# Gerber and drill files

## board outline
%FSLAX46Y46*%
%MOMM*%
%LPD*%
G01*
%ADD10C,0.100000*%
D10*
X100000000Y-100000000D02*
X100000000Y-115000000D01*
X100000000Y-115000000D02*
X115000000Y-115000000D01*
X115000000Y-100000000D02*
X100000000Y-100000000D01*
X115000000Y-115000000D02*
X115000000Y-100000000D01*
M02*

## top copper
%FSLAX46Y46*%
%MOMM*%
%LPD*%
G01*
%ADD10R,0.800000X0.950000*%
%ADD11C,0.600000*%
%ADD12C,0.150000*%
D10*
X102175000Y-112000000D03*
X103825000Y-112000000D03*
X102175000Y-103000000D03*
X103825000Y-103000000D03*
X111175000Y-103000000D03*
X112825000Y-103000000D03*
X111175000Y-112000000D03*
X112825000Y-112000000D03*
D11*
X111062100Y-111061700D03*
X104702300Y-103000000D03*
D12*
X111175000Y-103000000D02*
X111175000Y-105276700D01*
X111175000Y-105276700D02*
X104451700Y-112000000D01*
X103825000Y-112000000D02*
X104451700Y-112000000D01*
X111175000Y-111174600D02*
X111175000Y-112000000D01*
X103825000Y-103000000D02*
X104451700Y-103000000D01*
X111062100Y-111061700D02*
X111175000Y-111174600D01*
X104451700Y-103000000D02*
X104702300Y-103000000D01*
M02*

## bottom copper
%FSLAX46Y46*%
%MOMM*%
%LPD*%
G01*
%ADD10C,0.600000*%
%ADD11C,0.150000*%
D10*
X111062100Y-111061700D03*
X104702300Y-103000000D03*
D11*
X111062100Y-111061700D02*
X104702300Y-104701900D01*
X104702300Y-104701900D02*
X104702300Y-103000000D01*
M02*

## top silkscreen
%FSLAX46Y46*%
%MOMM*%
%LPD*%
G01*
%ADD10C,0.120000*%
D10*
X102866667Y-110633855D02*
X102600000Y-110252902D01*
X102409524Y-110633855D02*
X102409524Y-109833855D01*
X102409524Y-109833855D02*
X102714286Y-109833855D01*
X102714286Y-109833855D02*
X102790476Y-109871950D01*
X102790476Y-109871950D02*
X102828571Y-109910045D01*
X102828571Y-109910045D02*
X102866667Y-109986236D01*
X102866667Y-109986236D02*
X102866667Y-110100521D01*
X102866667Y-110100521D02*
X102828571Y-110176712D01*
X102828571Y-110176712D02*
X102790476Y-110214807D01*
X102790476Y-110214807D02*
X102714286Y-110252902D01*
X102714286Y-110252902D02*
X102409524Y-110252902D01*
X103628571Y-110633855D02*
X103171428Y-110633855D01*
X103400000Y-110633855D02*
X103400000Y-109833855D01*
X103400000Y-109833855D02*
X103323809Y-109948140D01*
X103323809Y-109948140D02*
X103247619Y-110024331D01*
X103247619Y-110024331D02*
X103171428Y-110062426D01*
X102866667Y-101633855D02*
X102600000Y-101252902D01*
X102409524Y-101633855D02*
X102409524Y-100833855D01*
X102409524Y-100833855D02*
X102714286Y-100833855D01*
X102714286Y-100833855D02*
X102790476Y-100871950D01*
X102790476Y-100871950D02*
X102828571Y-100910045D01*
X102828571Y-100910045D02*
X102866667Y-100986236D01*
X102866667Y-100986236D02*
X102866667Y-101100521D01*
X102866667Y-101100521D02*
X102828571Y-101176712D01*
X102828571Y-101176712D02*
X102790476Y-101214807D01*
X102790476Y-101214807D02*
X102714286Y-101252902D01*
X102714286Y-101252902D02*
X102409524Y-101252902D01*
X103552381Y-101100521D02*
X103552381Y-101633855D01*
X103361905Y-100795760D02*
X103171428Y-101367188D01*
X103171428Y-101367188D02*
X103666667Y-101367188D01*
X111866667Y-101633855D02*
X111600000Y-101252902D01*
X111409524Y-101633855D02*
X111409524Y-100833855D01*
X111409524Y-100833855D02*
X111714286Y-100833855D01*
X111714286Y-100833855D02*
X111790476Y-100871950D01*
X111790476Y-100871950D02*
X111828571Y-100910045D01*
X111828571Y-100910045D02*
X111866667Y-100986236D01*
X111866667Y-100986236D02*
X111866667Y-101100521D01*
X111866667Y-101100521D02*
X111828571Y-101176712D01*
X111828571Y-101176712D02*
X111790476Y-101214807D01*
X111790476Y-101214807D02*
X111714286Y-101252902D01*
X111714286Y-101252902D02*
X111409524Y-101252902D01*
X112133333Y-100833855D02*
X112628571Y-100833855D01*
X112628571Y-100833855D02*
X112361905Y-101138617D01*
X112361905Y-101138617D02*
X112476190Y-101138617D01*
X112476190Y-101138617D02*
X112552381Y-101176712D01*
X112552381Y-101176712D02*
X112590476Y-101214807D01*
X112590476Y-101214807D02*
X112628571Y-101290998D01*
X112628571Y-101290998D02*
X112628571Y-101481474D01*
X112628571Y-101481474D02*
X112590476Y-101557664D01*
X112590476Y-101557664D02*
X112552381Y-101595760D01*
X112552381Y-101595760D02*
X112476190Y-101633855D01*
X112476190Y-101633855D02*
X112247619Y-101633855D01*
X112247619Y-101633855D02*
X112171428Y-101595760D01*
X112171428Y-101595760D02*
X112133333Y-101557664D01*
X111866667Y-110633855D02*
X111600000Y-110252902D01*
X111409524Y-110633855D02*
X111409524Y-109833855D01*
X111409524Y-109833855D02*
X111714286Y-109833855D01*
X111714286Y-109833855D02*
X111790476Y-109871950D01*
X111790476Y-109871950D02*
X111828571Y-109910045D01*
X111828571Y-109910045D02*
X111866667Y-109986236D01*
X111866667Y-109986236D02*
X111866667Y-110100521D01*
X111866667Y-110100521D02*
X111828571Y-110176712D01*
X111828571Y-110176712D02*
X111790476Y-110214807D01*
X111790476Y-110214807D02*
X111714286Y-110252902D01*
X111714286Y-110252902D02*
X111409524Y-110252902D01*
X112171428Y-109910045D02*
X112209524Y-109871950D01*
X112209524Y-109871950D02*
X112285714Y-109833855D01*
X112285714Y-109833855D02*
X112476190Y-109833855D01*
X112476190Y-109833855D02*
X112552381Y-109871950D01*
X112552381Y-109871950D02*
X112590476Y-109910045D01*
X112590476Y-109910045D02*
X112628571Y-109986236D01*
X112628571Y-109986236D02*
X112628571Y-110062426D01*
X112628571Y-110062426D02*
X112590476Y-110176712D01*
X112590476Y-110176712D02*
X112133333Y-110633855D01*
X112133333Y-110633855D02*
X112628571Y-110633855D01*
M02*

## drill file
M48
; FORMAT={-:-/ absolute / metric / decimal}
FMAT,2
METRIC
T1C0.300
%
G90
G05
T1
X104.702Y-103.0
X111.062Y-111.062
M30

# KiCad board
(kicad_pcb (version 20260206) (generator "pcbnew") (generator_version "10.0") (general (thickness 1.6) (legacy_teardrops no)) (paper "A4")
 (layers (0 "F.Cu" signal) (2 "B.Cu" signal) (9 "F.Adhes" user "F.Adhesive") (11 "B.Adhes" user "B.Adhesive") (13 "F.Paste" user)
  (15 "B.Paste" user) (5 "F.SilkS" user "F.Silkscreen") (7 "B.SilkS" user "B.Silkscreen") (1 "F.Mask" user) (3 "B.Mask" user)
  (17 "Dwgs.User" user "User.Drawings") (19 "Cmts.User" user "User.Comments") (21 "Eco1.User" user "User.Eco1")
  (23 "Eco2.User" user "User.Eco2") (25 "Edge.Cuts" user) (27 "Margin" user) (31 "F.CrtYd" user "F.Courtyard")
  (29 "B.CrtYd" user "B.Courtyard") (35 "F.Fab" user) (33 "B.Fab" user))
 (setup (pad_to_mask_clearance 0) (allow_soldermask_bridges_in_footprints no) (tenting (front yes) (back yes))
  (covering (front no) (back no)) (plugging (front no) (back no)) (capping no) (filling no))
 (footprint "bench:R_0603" (layer "F.Cu") (at 103 112)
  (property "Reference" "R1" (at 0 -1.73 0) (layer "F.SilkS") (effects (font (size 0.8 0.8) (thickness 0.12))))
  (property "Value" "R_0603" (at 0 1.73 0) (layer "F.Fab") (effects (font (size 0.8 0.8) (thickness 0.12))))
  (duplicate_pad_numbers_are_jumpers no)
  (pad "1" smd rect (at -0.825 0) (size 0.8 0.95) (layers "F.Cu" "F.Mask" "F.Paste"))
  (pad "2" smd rect (at 0.825 0) (size 0.8 0.95) (layers "F.Cu" "F.Mask" "F.Paste") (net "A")))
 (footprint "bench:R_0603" (layer "F.Cu") (at 103 103)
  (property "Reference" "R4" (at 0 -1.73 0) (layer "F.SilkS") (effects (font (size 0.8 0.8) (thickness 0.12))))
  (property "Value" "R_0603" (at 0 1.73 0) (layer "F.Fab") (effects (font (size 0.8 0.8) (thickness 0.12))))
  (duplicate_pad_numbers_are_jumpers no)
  (pad "1" smd rect (at -0.825 0) (size 0.8 0.95) (layers "F.Cu" "F.Mask" "F.Paste"))
  (pad "2" smd rect (at 0.825 0) (size 0.8 0.95) (layers "F.Cu" "F.Mask" "F.Paste") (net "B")))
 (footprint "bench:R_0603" (layer "F.Cu") (at 112 103)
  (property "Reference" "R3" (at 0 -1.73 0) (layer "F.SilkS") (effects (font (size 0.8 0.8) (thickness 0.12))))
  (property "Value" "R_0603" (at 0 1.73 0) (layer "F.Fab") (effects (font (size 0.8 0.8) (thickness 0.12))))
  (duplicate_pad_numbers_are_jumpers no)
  (pad "1" smd rect (at -0.825 0) (size 0.8 0.95) (layers "F.Cu" "F.Mask" "F.Paste") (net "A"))
  (pad "2" smd rect (at 0.825 0) (size 0.8 0.95) (layers "F.Cu" "F.Mask" "F.Paste")))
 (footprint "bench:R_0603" (layer "F.Cu") (at 112 112)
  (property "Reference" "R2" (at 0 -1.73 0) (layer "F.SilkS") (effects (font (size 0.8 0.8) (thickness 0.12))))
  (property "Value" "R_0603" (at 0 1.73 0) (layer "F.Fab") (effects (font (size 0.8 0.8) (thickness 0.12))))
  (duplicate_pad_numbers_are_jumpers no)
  (pad "1" smd rect (at -0.825 0) (size 0.8 0.95) (layers "F.Cu" "F.Mask" "F.Paste") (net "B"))
  (pad "2" smd rect (at 0.825 0) (size 0.8 0.95) (layers "F.Cu" "F.Mask" "F.Paste")))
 (gr_line (start 100 100) (end 100 115) (stroke (width 0.1) (type solid)) (layer "Edge.Cuts"))
 (gr_line (start 100 115) (end 115 115) (stroke (width 0.1) (type solid)) (layer "Edge.Cuts"))
 (gr_line (start 115 100) (end 100 100) (stroke (width 0.1) (type solid)) (layer "Edge.Cuts"))
 (gr_line (start 115 115) (end 115 100) (stroke (width 0.1) (type solid)) (layer "Edge.Cuts"))
 (segment (start 111.175 103) (end 111.175 105.2767) (width 0.15) (layer "F.Cu") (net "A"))
 (segment (start 111.175 105.2767) (end 104.4517 112) (width 0.15) (layer "F.Cu") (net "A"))
 (segment (start 103.825 112) (end 104.4517 112) (width 0.15) (layer "F.Cu") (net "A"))
 (segment (start 111.175 111.1746) (end 111.175 112) (width 0.15) (layer "F.Cu") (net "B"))
 (segment (start 103.825 103) (end 104.4517 103) (width 0.15) (layer "F.Cu") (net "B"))
 (segment (start 111.0621 111.0617) (end 111.175 111.1746) (width 0.15) (layer "F.Cu") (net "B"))
 (segment (start 104.4517 103) (end 104.7023 103) (width 0.15) (layer "F.Cu") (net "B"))
 (via (at 111.0621 111.0617) (size 0.6) (drill 0.3) (layers "F.Cu" "B.Cu") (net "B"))
 (via (at 104.7023 103) (size 0.6) (drill 0.3) (layers "F.Cu" "B.Cu") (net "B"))
 (segment (start 111.0621 111.0617) (end 104.7023 104.7019) (width 0.15) (layer "B.Cu") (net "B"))
 (segment (start 104.7023 104.7019) (end 104.7023 103) (width 0.15) (layer "B.Cu") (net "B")))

